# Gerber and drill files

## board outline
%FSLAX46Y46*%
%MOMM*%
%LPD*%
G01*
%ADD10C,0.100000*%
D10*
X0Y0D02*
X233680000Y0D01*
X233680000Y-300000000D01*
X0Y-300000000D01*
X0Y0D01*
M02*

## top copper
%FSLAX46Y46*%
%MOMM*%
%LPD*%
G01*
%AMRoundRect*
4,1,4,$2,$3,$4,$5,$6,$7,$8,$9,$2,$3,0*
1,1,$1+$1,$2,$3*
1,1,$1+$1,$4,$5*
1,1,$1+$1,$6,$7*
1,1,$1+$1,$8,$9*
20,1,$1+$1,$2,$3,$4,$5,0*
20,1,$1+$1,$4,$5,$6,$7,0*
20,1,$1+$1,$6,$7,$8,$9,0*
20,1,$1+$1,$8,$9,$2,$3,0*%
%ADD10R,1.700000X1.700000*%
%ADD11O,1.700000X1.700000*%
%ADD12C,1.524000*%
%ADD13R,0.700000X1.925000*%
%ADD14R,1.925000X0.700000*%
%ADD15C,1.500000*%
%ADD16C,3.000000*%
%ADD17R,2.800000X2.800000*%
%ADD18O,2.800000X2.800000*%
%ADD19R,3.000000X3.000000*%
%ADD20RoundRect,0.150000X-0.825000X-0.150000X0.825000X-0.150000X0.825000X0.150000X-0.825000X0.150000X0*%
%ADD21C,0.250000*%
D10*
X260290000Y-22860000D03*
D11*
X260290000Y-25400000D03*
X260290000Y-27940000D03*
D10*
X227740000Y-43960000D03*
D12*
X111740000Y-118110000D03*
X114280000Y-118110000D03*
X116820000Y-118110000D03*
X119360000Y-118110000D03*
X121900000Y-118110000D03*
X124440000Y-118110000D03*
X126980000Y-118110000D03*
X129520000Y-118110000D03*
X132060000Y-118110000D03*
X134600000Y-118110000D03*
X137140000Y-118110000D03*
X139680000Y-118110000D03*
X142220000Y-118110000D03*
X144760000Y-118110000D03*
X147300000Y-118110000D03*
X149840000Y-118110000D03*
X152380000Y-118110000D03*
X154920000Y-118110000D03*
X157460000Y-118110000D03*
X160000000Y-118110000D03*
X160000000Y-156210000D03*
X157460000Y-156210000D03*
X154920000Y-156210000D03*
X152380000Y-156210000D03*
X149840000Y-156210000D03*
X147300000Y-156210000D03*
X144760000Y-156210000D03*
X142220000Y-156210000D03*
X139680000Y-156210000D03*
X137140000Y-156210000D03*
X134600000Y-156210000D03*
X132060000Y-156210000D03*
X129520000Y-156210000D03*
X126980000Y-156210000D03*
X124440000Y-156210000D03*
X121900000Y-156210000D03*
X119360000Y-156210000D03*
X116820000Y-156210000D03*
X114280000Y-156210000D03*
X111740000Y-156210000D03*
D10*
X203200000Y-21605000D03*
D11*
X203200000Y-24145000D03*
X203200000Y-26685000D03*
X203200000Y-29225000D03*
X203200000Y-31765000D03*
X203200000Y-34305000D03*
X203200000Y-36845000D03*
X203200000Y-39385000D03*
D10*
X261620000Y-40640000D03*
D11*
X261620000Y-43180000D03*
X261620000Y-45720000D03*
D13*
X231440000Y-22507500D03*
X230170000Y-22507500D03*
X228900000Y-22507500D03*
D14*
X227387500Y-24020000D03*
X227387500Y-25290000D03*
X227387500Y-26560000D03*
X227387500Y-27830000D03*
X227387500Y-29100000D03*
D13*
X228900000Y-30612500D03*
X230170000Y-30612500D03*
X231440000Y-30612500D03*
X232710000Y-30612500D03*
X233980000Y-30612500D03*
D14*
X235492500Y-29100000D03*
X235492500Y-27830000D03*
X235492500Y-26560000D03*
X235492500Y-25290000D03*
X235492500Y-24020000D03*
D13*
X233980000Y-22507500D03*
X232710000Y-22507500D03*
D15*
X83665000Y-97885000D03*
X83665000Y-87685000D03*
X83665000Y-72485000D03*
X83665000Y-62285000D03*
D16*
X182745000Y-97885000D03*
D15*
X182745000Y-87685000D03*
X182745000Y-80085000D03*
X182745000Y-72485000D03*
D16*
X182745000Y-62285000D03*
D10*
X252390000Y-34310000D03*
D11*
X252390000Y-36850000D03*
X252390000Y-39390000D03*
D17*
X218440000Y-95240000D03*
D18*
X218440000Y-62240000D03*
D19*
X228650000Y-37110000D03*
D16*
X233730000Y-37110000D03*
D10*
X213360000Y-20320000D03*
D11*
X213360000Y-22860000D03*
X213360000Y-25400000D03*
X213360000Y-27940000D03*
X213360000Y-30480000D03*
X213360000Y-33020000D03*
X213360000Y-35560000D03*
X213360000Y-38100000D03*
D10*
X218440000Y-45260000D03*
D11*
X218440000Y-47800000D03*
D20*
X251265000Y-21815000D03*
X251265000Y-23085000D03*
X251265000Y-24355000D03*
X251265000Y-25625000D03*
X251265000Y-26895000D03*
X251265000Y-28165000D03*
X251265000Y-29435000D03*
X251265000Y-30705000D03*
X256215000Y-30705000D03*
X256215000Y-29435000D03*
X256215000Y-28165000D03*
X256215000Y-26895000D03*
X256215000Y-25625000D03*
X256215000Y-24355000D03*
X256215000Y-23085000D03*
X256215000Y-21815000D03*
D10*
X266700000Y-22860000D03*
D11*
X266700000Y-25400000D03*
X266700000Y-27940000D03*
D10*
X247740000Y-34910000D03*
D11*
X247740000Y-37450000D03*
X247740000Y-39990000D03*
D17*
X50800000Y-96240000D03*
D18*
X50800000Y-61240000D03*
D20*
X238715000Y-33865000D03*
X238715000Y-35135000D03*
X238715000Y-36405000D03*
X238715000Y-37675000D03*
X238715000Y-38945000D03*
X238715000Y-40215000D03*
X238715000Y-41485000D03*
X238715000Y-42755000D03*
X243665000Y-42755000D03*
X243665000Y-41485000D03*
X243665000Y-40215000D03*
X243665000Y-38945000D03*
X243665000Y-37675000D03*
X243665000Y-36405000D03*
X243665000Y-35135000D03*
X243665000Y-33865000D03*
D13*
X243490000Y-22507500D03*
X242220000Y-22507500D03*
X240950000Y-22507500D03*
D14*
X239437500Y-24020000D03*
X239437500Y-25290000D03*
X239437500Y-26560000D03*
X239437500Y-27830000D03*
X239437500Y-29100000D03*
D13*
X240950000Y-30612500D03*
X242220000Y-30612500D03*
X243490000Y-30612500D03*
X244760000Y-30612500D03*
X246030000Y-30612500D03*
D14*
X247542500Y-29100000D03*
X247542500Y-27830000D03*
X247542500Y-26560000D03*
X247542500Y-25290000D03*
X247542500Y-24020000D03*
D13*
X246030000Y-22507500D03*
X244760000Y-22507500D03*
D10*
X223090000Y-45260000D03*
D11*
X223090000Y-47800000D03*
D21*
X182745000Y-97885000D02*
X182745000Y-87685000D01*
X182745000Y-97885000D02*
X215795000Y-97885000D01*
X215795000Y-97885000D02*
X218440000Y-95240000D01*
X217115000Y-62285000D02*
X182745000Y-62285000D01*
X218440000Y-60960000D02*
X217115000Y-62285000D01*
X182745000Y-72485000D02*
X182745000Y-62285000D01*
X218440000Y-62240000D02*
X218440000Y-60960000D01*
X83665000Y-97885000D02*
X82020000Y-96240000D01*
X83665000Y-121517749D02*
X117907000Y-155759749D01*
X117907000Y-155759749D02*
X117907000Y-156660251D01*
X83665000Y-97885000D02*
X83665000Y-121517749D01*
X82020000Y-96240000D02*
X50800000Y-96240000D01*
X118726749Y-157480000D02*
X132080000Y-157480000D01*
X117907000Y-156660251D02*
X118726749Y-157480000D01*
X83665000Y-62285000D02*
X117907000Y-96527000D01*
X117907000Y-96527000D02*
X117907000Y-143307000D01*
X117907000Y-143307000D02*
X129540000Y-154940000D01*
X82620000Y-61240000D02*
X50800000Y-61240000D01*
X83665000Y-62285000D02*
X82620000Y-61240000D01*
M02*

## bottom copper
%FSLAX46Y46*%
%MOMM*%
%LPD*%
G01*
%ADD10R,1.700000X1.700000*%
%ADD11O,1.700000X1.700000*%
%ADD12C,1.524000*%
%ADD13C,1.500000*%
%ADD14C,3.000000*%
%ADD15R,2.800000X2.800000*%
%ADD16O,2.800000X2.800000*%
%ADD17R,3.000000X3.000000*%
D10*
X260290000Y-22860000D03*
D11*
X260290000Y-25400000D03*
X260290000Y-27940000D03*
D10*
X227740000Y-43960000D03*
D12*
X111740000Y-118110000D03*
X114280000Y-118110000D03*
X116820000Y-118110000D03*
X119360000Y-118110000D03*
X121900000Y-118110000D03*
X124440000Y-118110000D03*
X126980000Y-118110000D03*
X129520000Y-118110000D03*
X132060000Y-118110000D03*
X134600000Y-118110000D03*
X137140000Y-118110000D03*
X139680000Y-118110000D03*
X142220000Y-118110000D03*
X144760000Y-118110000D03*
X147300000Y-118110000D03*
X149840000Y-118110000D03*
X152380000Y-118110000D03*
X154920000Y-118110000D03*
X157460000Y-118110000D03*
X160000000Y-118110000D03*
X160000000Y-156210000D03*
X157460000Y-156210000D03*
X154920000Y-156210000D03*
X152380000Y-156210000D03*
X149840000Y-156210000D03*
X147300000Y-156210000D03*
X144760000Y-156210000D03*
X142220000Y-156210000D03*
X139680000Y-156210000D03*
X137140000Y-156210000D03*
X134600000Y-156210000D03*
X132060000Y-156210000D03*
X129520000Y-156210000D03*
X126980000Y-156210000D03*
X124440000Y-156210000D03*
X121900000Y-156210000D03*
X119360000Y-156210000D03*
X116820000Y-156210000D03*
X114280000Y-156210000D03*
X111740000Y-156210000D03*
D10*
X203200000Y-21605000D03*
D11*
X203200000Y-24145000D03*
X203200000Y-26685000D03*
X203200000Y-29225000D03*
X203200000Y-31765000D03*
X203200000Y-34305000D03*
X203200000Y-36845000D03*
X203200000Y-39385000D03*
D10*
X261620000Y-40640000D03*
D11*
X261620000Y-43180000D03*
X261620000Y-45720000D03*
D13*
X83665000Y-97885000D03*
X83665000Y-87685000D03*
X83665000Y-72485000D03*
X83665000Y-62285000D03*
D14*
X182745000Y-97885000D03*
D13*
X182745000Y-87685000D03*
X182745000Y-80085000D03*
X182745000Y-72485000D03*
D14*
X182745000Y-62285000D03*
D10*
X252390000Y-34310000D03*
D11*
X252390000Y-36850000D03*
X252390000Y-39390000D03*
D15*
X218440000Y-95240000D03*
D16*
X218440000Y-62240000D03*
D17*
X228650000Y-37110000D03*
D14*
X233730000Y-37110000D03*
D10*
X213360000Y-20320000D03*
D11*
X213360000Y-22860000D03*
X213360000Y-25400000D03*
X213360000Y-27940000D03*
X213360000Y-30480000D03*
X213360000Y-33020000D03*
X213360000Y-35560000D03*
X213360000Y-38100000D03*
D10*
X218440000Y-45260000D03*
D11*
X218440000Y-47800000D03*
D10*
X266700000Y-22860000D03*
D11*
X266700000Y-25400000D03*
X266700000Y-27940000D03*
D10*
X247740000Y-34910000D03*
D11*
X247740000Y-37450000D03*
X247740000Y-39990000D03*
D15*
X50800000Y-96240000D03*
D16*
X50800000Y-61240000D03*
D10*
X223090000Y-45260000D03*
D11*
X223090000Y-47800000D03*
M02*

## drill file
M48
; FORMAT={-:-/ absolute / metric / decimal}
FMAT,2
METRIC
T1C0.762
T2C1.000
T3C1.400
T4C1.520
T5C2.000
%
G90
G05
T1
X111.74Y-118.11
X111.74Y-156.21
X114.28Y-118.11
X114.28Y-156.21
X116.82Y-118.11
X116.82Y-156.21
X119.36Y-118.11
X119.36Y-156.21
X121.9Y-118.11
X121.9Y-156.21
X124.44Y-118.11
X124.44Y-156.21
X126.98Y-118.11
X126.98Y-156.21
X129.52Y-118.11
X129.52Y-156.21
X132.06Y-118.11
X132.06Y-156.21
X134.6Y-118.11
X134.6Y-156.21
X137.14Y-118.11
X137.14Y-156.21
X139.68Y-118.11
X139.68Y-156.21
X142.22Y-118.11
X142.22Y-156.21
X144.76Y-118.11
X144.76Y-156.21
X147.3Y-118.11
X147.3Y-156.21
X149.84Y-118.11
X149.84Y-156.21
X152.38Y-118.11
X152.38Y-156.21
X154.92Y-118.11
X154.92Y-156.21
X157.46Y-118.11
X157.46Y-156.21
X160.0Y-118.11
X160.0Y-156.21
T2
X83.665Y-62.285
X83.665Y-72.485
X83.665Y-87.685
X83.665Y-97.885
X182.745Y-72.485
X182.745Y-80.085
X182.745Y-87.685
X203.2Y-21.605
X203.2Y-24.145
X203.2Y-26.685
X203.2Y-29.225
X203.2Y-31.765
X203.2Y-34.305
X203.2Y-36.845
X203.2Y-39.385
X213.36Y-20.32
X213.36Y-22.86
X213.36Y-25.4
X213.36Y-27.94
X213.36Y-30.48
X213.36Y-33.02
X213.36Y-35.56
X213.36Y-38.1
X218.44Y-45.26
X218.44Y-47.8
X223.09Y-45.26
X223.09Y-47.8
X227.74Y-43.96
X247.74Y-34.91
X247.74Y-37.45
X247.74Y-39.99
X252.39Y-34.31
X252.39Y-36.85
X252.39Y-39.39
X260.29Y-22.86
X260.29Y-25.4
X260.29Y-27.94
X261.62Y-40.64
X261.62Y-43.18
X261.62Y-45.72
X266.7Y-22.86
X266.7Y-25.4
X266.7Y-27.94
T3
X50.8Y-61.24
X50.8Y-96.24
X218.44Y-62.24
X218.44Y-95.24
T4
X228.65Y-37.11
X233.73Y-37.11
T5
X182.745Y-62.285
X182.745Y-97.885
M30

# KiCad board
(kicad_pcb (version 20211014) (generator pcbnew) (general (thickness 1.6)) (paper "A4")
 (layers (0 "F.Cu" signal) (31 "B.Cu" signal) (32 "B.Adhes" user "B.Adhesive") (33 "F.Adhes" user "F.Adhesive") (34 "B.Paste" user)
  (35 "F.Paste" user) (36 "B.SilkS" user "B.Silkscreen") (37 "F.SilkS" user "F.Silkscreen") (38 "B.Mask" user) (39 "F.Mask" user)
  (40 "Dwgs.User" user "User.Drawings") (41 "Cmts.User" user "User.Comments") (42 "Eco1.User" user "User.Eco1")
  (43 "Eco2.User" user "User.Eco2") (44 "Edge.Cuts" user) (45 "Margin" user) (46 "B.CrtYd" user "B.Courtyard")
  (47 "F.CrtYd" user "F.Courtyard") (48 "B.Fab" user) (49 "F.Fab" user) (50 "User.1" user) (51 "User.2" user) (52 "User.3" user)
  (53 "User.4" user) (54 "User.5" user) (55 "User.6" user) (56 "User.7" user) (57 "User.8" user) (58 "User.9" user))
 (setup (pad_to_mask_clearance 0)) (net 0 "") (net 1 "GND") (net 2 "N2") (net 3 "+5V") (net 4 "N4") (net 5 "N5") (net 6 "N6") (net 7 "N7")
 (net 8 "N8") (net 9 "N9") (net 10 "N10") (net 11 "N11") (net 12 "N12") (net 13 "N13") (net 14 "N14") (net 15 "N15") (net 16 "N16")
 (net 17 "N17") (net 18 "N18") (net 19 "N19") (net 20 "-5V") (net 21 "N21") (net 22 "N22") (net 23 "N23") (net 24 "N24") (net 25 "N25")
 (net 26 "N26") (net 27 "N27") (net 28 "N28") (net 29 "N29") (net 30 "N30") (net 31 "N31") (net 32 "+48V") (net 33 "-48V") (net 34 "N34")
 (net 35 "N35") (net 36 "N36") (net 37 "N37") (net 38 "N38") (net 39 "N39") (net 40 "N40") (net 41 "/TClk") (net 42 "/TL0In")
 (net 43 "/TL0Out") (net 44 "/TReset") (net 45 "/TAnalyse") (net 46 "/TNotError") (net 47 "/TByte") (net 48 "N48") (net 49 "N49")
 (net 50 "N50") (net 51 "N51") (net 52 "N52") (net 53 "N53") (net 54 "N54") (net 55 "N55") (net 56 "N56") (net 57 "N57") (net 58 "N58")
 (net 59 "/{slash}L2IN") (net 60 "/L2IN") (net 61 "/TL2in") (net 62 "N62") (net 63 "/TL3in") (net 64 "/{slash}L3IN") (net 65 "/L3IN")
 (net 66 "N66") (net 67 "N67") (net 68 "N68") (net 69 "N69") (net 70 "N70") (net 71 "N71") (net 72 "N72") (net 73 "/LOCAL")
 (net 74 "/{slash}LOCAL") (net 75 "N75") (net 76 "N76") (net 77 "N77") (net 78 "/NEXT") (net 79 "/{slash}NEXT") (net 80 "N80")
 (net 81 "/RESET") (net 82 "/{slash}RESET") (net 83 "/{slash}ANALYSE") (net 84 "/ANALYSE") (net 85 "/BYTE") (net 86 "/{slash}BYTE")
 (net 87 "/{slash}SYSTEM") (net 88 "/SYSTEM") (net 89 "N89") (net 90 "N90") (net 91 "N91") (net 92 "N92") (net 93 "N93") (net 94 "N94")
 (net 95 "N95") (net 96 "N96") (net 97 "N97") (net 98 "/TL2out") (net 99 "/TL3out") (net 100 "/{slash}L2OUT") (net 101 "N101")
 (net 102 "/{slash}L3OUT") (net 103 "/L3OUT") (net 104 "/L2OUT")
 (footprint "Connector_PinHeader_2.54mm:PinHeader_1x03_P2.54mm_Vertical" (layer "F.Cu") (at 260.29 22.86)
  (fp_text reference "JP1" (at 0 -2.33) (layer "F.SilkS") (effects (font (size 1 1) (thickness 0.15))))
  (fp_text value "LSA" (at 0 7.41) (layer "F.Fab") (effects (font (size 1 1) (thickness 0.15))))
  (pad "1" thru_hole rect (at 0 0) (size 1.7 1.7) (drill 1) (layers *.Cu *.Mask) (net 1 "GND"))
  (pad "2" thru_hole oval (at 0 2.54) (size 1.7 1.7) (drill 1) (layers *.Cu *.Mask) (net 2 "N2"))
  (pad "3" thru_hole oval (at 0 5.08) (size 1.7 1.7) (drill 1) (layers *.Cu *.Mask) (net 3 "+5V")))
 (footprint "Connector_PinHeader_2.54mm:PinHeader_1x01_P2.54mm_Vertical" (layer "F.Cu") (at 227.74 43.96)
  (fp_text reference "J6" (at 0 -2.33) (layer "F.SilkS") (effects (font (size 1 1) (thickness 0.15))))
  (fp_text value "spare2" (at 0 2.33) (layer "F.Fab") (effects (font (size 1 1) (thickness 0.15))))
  (pad "1" thru_hole rect (at 0 0) (size 1.7 1.7) (drill 1) (layers *.Cu *.Mask) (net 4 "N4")))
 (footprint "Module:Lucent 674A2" (layer "F.Cu") (at 137.16 137.16)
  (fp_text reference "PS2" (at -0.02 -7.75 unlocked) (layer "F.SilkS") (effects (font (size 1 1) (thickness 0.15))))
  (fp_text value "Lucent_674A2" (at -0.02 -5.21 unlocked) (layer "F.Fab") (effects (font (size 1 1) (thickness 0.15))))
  (pad "1" thru_hole circle (at -25.42 -19.05) (size 1.524 1.524) (drill 0.762) (layers *.Cu *.Mask) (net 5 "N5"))
  (pad "2" thru_hole circle (at -22.88 -19.05) (size 1.524 1.524) (drill 0.762) (layers *.Cu *.Mask) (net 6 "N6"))
  (pad "3" thru_hole circle (at -20.34 -19.05) (size 1.524 1.524) (drill 0.762) (layers *.Cu *.Mask) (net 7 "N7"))
  (pad "4" thru_hole circle (at -17.8 -19.05) (size 1.524 1.524) (drill 0.762) (layers *.Cu *.Mask) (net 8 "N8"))
  (pad "5" thru_hole circle (at -15.26 -19.05) (size 1.524 1.524) (drill 0.762) (layers *.Cu *.Mask) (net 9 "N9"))
  (pad "6" thru_hole circle (at -12.72 -19.05) (size 1.524 1.524) (drill 0.762) (layers *.Cu *.Mask) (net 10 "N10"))
  (pad "7" thru_hole circle (at -10.18 -19.05) (size 1.524 1.524) (drill 0.762) (layers *.Cu *.Mask) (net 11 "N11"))
  (pad "8" thru_hole circle (at -7.64 -19.05) (size 1.524 1.524) (drill 0.762) (layers *.Cu *.Mask) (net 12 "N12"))
  (pad "9" thru_hole circle (at -5.1 -19.05) (size 1.524 1.524) (drill 0.762) (layers *.Cu *.Mask) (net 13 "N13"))
  (pad "10" thru_hole circle (at -2.56 -19.05) (size 1.524 1.524) (drill 0.762) (layers *.Cu *.Mask) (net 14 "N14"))
  (pad "11" thru_hole circle (at -0.02 -19.05) (size 1.524 1.524) (drill 0.762) (layers *.Cu *.Mask) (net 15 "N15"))
  (pad "12" thru_hole circle (at 2.52 -19.05) (size 1.524 1.524) (drill 0.762) (layers *.Cu *.Mask) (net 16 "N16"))
  (pad "13" thru_hole circle (at 5.06 -19.05) (size 1.524 1.524) (drill 0.762) (layers *.Cu *.Mask) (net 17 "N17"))
  (pad "14" thru_hole circle (at 7.6 -19.05) (size 1.524 1.524) (drill 0.762) (layers *.Cu *.Mask) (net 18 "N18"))
  (pad "15" thru_hole circle (at 10.14 -19.05) (size 1.524 1.524) (drill 0.762) (layers *.Cu *.Mask) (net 18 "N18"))
  (pad "16" thru_hole circle (at 12.68 -19.05) (size 1.524 1.524) (drill 0.762) (layers *.Cu *.Mask) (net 18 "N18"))
  (pad "17" thru_hole circle (at 15.22 -19.05) (size 1.524 1.524) (drill 0.762) (layers *.Cu *.Mask) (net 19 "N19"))
  (pad "18" thru_hole circle (at 17.76 -19.05) (size 1.524 1.524) (drill 0.762) (layers *.Cu *.Mask) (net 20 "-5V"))
  (pad "19" thru_hole circle (at 20.3 -19.05) (size 1.524 1.524) (drill 0.762) (layers *.Cu *.Mask) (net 20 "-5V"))
  (pad "20" thru_hole circle (at 22.84 -19.05) (size 1.524 1.524) (drill 0.762) (layers *.Cu *.Mask) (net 20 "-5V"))
  (pad "21" thru_hole circle (at 22.84 19.05) (size 1.524 1.524) (drill 0.762) (layers *.Cu *.Mask) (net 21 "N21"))
  (pad "22" thru_hole circle (at 20.3 19.05) (size 1.524 1.524) (drill 0.762) (layers *.Cu *.Mask) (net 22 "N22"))
  (pad "23" thru_hole circle (at 17.76 19.05) (size 1.524 1.524) (drill 0.762) (layers *.Cu *.Mask) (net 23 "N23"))
  (pad "24" thru_hole circle (at 15.22 19.05) (size 1.524 1.524) (drill 0.762) (layers *.Cu *.Mask) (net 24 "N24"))
  (pad "25" thru_hole circle (at 12.68 19.05) (size 1.524 1.524) (drill 0.762) (layers *.Cu *.Mask) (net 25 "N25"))
  (pad "26" thru_hole circle (at 10.14 19.05) (size 1.524 1.524) (drill 0.762) (layers *.Cu *.Mask) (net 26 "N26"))
  (pad "27" thru_hole circle (at 7.6 19.05) (size 1.524 1.524) (drill 0.762) (layers *.Cu *.Mask) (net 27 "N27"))
  (pad "28" thru_hole circle (at 5.06 19.05) (size 1.524 1.524) (drill 0.762) (layers *.Cu *.Mask) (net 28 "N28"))
  (pad "29" thru_hole circle (at 2.52 19.05) (size 1.524 1.524) (drill 0.762) (layers *.Cu *.Mask) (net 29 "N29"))
  (pad "30" thru_hole circle (at -0.02 19.05) (size 1.524 1.524) (drill 0.762) (layers *.Cu *.Mask) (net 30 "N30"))
  (pad "31" thru_hole circle (at -2.56 19.05) (size 1.524 1.524) (drill 0.762) (layers *.Cu *.Mask) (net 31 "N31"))
  (pad "32" thru_hole circle (at -5.1 19.05) (size 1.524 1.524) (drill 0.762) (layers *.Cu *.Mask) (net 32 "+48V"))
  (pad "33" thru_hole circle (at -7.64 19.05) (size 1.524 1.524) (drill 0.762) (layers *.Cu *.Mask) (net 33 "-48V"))
  (pad "34" thru_hole circle (at -10.18 19.05) (size 1.524 1.524) (drill 0.762) (layers *.Cu *.Mask) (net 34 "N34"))
  (pad "35" thru_hole circle (at -12.72 19.05) (size 1.524 1.524) (drill 0.762) (layers *.Cu *.Mask) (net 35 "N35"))
  (pad "36" thru_hole circle (at -15.26 19.05) (size 1.524 1.524) (drill 0.762) (layers *.Cu *.Mask) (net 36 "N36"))
  (pad "37" thru_hole circle (at -17.8 19.05) (size 1.524 1.524) (drill 0.762) (layers *.Cu *.Mask) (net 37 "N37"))
  (pad "38" thru_hole circle (at -20.34 19.05) (size 1.524 1.524) (drill 0.762) (layers *.Cu *.Mask) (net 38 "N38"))
  (pad "39" thru_hole circle (at -22.88 19.05) (size 1.524 1.524) (drill 0.762) (layers *.Cu *.Mask) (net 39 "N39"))
  (pad "40" thru_hole circle (at -25.42 19.05) (size 1.524 1.524) (drill 0.762) (layers *.Cu *.Mask) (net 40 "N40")))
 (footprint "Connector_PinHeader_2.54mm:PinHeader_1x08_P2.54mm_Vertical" (layer "F.Cu") (at 203.2 21.605)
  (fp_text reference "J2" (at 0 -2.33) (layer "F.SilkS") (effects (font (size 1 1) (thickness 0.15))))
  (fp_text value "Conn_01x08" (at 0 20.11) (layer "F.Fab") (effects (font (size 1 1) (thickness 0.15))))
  (pad "1" thru_hole rect (at 0 0) (size 1.7 1.7) (drill 1) (layers *.Cu *.Mask) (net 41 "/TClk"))
  (pad "2" thru_hole oval (at 0 2.54) (size 1.7 1.7) (drill 1) (layers *.Cu *.Mask) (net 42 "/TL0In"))
  (pad "3" thru_hole oval (at 0 5.08) (size 1.7 1.7) (drill 1) (layers *.Cu *.Mask) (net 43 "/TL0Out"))
  (pad "4" thru_hole oval (at 0 7.62) (size 1.7 1.7) (drill 1) (layers *.Cu *.Mask) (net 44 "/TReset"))
  (pad "5" thru_hole oval (at 0 10.16) (size 1.7 1.7) (drill 1) (layers *.Cu *.Mask) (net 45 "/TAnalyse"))
  (pad "6" thru_hole oval (at 0 12.7) (size 1.7 1.7) (drill 1) (layers *.Cu *.Mask) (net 1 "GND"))
  (pad "7" thru_hole oval (at 0 15.24) (size 1.7 1.7) (drill 1) (layers *.Cu *.Mask) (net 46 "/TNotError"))
  (pad "8" thru_hole oval (at 0 17.78) (size 1.7 1.7) (drill 1) (layers *.Cu *.Mask) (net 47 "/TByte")))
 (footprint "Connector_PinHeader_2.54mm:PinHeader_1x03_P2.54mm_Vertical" (layer "F.Cu") (at 261.62 40.64)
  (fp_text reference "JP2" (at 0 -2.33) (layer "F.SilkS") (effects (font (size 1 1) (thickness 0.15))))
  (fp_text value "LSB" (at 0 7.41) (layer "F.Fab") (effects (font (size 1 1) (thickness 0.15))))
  (pad "1" thru_hole rect (at 0 0) (size 1.7 1.7) (drill 1) (layers *.Cu *.Mask) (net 1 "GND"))
  (pad "2" thru_hole oval (at 0 2.54) (size 1.7 1.7) (drill 1) (layers *.Cu *.Mask) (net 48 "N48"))
  (pad "3" thru_hole oval (at 0 5.08) (size 1.7 1.7) (drill 1) (layers *.Cu *.Mask) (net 3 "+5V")))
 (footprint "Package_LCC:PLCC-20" (layer "F.Cu") (at 231.44 26.56)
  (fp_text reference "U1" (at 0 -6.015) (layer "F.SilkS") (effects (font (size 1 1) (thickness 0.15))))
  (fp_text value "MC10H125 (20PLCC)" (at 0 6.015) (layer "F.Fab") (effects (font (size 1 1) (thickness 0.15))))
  (pad "1" smd rect (at 0 -4.0525) (size 0.7 1.925) (layers "F.Cu" "F.Paste" "F.Mask") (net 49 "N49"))
  (pad "2" smd rect (at -1.27 -4.0525) (size 0.7 1.925) (layers "F.Cu" "F.Paste" "F.Mask") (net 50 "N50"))
  (pad "3" smd rect (at -2.54 -4.0525) (size 0.7 1.925) (layers "F.Cu" "F.Paste" "F.Mask") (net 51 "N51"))
  (pad "4" smd rect (at -4.0525 -2.54) (size 1.925 0.7) (layers "F.Cu" "F.Paste" "F.Mask") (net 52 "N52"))
  (pad "5" smd rect (at -4.0525 -1.27) (size 1.925 0.7) (layers "F.Cu" "F.Paste" "F.Mask") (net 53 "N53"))
  (pad "6" smd rect (at -4.0525 0) (size 1.925 0.7) (layers "F.Cu" "F.Paste" "F.Mask") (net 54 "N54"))
  (pad "7" smd rect (at -4.0525 1.27) (size 1.925 0.7) (layers "F.Cu" "F.Paste" "F.Mask") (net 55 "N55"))
  (pad "8" smd rect (at -4.0525 2.54) (size 1.925 0.7) (layers "F.Cu" "F.Paste" "F.Mask") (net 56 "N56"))
  (pad "9" smd rect (at -2.54 4.0525) (size 0.7 1.925) (layers "F.Cu" "F.Paste" "F.Mask") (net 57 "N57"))
  (pad "10" smd rect (at -1.27 4.0525) (size 0.7 1.925) (layers "F.Cu" "F.Paste" "F.Mask") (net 20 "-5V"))
  (pad "11" smd rect (at 0 4.0525) (size 0.7 1.925) (layers "F.Cu" "F.Paste" "F.Mask") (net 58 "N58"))
  (pad "12" smd rect (at 1.27 4.0525) (size 0.7 1.925) (layers "F.Cu" "F.Paste" "F.Mask") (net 3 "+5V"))
  (pad "13" smd rect (at 2.54 4.0525) (size 0.7 1.925) (layers "F.Cu" "F.Paste" "F.Mask") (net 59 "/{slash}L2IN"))
  (pad "14" smd rect (at 4.0525 2.54) (size 1.925 0.7) (layers "F.Cu" "F.Paste" "F.Mask") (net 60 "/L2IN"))
  (pad "15" smd rect (at 4.0525 1.27) (size 1.925 0.7) (layers "F.Cu" "F.Paste" "F.Mask") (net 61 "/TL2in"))
  (pad "16" smd rect (at 4.0525 0) (size 1.925 0.7) (layers "F.Cu" "F.Paste" "F.Mask") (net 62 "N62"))
  (pad "17" smd rect (at 4.0525 -1.27) (size 1.925 0.7) (layers "F.Cu" "F.Paste" "F.Mask") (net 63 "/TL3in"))
  (pad "18" smd rect (at 4.0525 -2.54) (size 1.925 0.7) (layers "F.Cu" "F.Paste" "F.Mask") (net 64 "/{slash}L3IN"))
  (pad "19" smd rect (at 2.54 -4.0525) (size 0.7 1.925) (layers "F.Cu" "F.Paste" "F.Mask") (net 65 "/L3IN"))
  (pad "20" smd rect (at 1.27 -4.0525) (size 0.7 1.925) (layers "F.Cu" "F.Paste" "F.Mask") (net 1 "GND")))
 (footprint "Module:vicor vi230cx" (layer "F.Cu") (at 76.065 49.585)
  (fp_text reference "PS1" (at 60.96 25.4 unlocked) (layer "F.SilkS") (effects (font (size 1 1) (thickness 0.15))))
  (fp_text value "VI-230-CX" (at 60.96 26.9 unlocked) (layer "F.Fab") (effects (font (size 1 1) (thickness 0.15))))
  (pad "1" thru_hole circle (at 7.6 48.3) (size 1.5 1.5) (drill 1) (layers *.Cu *.Mask) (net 32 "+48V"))
  (pad "2" thru_hole circle (at 7.6 38.1) (size 1.5 1.5) (drill 1) (layers *.Cu *.Mask) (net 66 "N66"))
  (pad "3" thru_hole circle (at 7.6 22.9) (size 1.5 1.5) (drill 1) (layers *.Cu *.Mask) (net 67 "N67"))
  (pad "4" thru_hole circle (at 7.6 12.7) (size 1.5 1.5) (drill 1) (layers *.Cu *.Mask) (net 33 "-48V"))
  (pad "5" thru_hole circle (at 106.68 48.3) (size 3 3) (drill 2) (layers *.Cu *.Mask) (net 3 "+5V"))
  (pad "6" thru_hole circle (at 106.68 38.1) (size 1.5 1.5) (drill 1) (layers *.Cu *.Mask) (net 3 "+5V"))
  (pad "7" thru_hole circle (at 106.68 30.5) (size 1.5 1.5) (drill 1) (layers *.Cu *.Mask) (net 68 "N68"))
  (pad "8" thru_hole circle (at 106.68 22.9) (size 1.5 1.5) (drill 1) (layers *.Cu *.Mask) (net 1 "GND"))
  (pad "9" thru_hole circle (at 106.68 12.7) (size 3 3) (drill 2) (layers *.Cu *.Mask) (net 1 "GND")))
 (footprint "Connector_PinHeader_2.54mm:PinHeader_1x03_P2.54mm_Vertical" (layer "F.Cu") (at 252.39 34.31)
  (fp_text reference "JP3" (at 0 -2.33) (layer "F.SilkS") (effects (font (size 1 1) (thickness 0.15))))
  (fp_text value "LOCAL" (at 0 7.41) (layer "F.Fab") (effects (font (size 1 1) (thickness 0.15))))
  (pad "1" thru_hole rect (at 0 0) (size 1.7 1.7) (drill 1) (layers *.Cu *.Mask) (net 1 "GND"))
  (pad "2" thru_hole oval (at 0 2.54) (size 1.7 1.7) (drill 1) (layers *.Cu *.Mask) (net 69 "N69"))
  (pad "3" thru_hole oval (at 0 5.08) (size 1.7 1.7) (drill 1) (layers *.Cu *.Mask) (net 3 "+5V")))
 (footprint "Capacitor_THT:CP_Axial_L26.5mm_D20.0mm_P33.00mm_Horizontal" (layer "F.Cu") (at 218.44 95.24 90)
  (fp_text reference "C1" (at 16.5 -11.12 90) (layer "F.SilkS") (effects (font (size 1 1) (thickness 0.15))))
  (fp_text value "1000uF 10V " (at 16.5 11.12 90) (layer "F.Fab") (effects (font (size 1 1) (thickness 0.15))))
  (pad "1" thru_hole rect (at 0 0 90) (size 2.8 2.8) (drill 1.4) (layers *.Cu *.Mask) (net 3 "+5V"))
  (pad "2" thru_hole oval (at 33 0 90) (size 2.8 2.8) (drill 1.4) (layers *.Cu *.Mask) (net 1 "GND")))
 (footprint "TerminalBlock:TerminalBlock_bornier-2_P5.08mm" (layer "F.Cu") (at 228.65 37.11)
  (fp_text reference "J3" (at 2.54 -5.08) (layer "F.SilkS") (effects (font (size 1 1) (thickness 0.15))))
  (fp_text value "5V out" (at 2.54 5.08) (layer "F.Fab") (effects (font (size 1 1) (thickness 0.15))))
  (pad "1" thru_hole rect (at 0 0) (size 3 3) (drill 1.52) (layers *.Cu *.Mask) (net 1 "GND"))
  (pad "2" thru_hole circle (at 5.08 0) (size 3 3) (drill 1.52) (layers *.Cu *.Mask) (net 3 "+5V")))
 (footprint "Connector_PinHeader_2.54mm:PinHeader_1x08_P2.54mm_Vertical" (layer "F.Cu") (at 213.36 20.32)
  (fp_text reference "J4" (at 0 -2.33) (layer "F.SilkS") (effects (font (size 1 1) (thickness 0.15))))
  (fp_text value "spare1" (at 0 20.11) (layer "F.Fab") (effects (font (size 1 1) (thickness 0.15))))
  (pad "1" thru_hole rect (at 0 0) (size 1.7 1.7) (drill 1) (layers *.Cu *.Mask) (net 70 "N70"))
  (pad "2" thru_hole oval (at 0 2.54) (size 1.7 1.7) (drill 1) (layers *.Cu *.Mask))
  (pad "3" thru_hole oval (at 0 5.08) (size 1.7 1.7) (drill 1) (layers *.Cu *.Mask))
  (pad "4" thru_hole oval (at 0 7.62) (size 1.7 1.7) (drill 1) (layers *.Cu *.Mask))
  (pad "5" thru_hole oval (at 0 10.16) (size 1.7 1.7) (drill 1) (layers *.Cu *.Mask))
  (pad "6" thru_hole oval (at 0 12.7) (size 1.7 1.7) (drill 1) (layers *.Cu *.Mask))
  (pad "7" thru_hole oval (at 0 15.24) (size 1.7 1.7) (drill 1) (layers *.Cu *.Mask))
  (pad "8" thru_hole oval (at 0 17.78) (size 1.7 1.7) (drill 1) (layers *.Cu *.Mask)))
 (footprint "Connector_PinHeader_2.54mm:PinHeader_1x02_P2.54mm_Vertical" (layer "F.Cu") (at 218.44 45.26)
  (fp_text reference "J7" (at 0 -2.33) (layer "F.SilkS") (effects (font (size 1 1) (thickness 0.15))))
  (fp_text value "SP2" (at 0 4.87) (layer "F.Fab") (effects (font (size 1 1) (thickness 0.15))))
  (pad "1" thru_hole rect (at 0 0) (size 1.7 1.7) (drill 1) (layers *.Cu *.Mask) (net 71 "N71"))
  (pad "2" thru_hole oval (at 0 2.54) (size 1.7 1.7) (drill 1) (layers *.Cu *.Mask) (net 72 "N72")))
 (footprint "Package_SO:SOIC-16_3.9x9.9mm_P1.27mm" (layer "F.Cu") (at 253.74 26.26)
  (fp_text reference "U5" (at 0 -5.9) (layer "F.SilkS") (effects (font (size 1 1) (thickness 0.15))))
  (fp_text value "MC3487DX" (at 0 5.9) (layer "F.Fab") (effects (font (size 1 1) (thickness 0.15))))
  (pad "1" smd roundrect (at -2.475 -4.445) (size 1.95 0.6) (layers "F.Cu" "F.Paste" "F.Mask") (roundrect_rratio 0.25) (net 69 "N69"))
  (pad "2" smd roundrect (at -2.475 -3.175) (size 1.95 0.6) (layers "F.Cu" "F.Paste" "F.Mask") (roundrect_rratio 0.25) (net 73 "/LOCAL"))
  (pad "3" smd roundrect (at -2.475 -1.905) (size 1.95 0.6) (layers "F.Cu" "F.Paste" "F.Mask") (roundrect_rratio 0.25)
   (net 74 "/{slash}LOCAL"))
  (pad "4" smd roundrect (at -2.475 -0.635) (size 1.95 0.6) (layers "F.Cu" "F.Paste" "F.Mask") (roundrect_rratio 0.25) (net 3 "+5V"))
  (pad "5" smd roundrect (at -2.475 0.635) (size 1.95 0.6) (layers "F.Cu" "F.Paste" "F.Mask") (roundrect_rratio 0.25) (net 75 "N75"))
  (pad "6" smd roundrect (at -2.475 1.905) (size 1.95 0.6) (layers "F.Cu" "F.Paste" "F.Mask") (roundrect_rratio 0.25) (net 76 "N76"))
  (pad "7" smd roundrect (at -2.475 3.175) (size 1.95 0.6) (layers "F.Cu" "F.Paste" "F.Mask") (roundrect_rratio 0.25) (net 70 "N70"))
  (pad "8" smd roundrect (at -2.475 4.445) (size 1.95 0.6) (layers "F.Cu" "F.Paste" "F.Mask") (roundrect_rratio 0.25) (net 1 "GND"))
  (pad "9" smd roundrect (at 2.475 4.445) (size 1.95 0.6) (layers "F.Cu" "F.Paste" "F.Mask") (roundrect_rratio 0.25) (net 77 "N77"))
  (pad "10" smd roundrect (at 2.475 3.175) (size 1.95 0.6) (layers "F.Cu" "F.Paste" "F.Mask") (roundrect_rratio 0.25) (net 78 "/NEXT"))
  (pad "11" smd roundrect (at 2.475 1.905) (size 1.95 0.6) (layers "F.Cu" "F.Paste" "F.Mask") (roundrect_rratio 0.25)
   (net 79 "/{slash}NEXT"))
  (pad "12" smd roundrect (at 2.475 0.635) (size 1.95 0.6) (layers "F.Cu" "F.Paste" "F.Mask") (roundrect_rratio 0.25) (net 3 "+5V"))
  (pad "13" smd roundrect (at 2.475 -0.635) (size 1.95 0.6) (layers "F.Cu" "F.Paste" "F.Mask") (roundrect_rratio 0.25) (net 71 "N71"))
  (pad "14" smd roundrect (at 2.475 -1.905) (size 1.95 0.6) (layers "F.Cu" "F.Paste" "F.Mask") (roundrect_rratio 0.25) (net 72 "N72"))
  (pad "15" smd roundrect (at 2.475 -3.175) (size 1.95 0.6) (layers "F.Cu" "F.Paste" "F.Mask") (roundrect_rratio 0.25) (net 4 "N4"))
  (pad "16" smd roundrect (at 2.475 -4.445) (size 1.95 0.6) (layers "F.Cu" "F.Paste" "F.Mask") (roundrect_rratio 0.25) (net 3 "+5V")))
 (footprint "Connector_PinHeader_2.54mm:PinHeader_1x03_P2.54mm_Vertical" (layer "F.Cu") (at 266.7 22.86)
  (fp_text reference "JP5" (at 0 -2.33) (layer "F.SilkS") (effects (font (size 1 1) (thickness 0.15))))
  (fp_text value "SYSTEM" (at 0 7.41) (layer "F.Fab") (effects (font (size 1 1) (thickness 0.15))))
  (pad "1" thru_hole rect (at 0 0) (size 1.7 1.7) (drill 1) (layers *.Cu *.Mask) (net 1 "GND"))
  (pad "2" thru_hole oval (at 0 2.54) (size 1.7 1.7) (drill 1) (layers *.Cu *.Mask) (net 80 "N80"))
  (pad "3" thru_hole oval (at 0 5.08) (size 1.7 1.7) (drill 1) (layers *.Cu *.Mask) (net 3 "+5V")))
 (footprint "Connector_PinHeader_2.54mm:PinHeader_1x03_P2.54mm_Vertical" (layer "F.Cu") (at 247.74 34.91)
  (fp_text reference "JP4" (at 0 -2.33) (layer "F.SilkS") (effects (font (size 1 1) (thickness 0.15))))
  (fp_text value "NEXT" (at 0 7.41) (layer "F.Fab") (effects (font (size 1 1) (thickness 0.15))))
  (pad "1" thru_hole rect (at 0 0) (size 1.7 1.7) (drill 1) (layers *.Cu *.Mask) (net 1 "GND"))
  (pad "2" thru_hole oval (at 0 2.54) (size 1.7 1.7) (drill 1) (layers *.Cu *.Mask) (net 77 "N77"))
  (pad "3" thru_hole oval (at 0 5.08) (size 1.7 1.7) (drill 1) (layers *.Cu *.Mask) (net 3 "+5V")))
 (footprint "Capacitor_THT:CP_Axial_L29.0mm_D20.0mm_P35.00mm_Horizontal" (layer "F.Cu") (at 50.8 96.24 90)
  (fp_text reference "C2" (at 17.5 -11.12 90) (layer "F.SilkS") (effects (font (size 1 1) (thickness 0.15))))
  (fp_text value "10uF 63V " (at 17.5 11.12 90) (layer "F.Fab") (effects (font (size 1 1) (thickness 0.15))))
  (pad "1" thru_hole rect (at 0 0 90) (size 2.8 2.8) (drill 1.4) (layers *.Cu *.Mask) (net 32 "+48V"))
  (pad "2" thru_hole oval (at 35 0 90) (size 2.8 2.8) (drill 1.4) (layers *.Cu *.Mask) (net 33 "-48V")))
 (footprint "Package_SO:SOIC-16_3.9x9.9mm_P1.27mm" (layer "F.Cu") (at 241.19 38.31)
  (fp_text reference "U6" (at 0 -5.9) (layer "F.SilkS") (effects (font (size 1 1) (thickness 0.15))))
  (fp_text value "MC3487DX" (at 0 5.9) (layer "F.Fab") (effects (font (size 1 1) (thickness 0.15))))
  (pad "1" smd roundrect (at -2.475 -4.445) (size 1.95 0.6) (layers "F.Cu" "F.Paste" "F.Mask") (roundrect_rratio 0.25) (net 44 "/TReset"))
  (pad "2" smd roundrect (at -2.475 -3.175) (size 1.95 0.6) (layers "F.Cu" "F.Paste" "F.Mask") (roundrect_rratio 0.25) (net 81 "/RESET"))
  (pad "3" smd roundrect (at -2.475 -1.905) (size 1.95 0.6) (layers "F.Cu" "F.Paste" "F.Mask") (roundrect_rratio 0.25)
   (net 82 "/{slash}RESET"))
  (pad "4" smd roundrect (at -2.475 -0.635) (size 1.95 0.6) (layers "F.Cu" "F.Paste" "F.Mask") (roundrect_rratio 0.25) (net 3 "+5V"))
  (pad "5" smd roundrect (at -2.475 0.635) (size 1.95 0.6) (layers "F.Cu" "F.Paste" "F.Mask") (roundrect_rratio 0.25)
   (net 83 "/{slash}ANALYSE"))
  (pad "6" smd roundrect (at -2.475 1.905) (size 1.95 0.6) (layers "F.Cu" "F.Paste" "F.Mask") (roundrect_rratio 0.25) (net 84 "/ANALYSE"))
  (pad "7" smd roundrect (at -2.475 3.175) (size 1.95 0.6) (layers "F.Cu" "F.Paste" "F.Mask") (roundrect_rratio 0.25) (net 45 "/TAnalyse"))
  (pad "8" smd roundrect (at -2.475 4.445) (size 1.95 0.6) (layers "F.Cu" "F.Paste" "F.Mask") (roundrect_rratio 0.25) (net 1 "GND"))
  (pad "9" smd roundrect (at 2.475 4.445) (size 1.95 0.6) (layers "F.Cu" "F.Paste" "F.Mask") (roundrect_rratio 0.25) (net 47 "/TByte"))
  (pad "10" smd roundrect (at 2.475 3.175) (size 1.95 0.6) (layers "F.Cu" "F.Paste" "F.Mask") (roundrect_rratio 0.25) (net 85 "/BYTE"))
  (pad "11" smd roundrect (at 2.475 1.905) (size 1.95 0.6) (layers "F.Cu" "F.Paste" "F.Mask") (roundrect_rratio 0.25)
   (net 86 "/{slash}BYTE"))
  (pad "12" smd roundrect (at 2.475 0.635) (size 1.95 0.6) (layers "F.Cu" "F.Paste" "F.Mask") (roundrect_rratio 0.25) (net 3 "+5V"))
  (pad "13" smd roundrect (at 2.475 -0.635) (size 1.95 0.6) (layers "F.Cu" "F.Paste" "F.Mask") (roundrect_rratio 0.25)
   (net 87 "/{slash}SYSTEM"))
  (pad "14" smd roundrect (at 2.475 -1.905) (size 1.95 0.6) (layers "F.Cu" "F.Paste" "F.Mask") (roundrect_rratio 0.25) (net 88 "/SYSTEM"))
  (pad "15" smd roundrect (at 2.475 -3.175) (size 1.95 0.6) (layers "F.Cu" "F.Paste" "F.Mask") (roundrect_rratio 0.25) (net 80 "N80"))
  (pad "16" smd roundrect (at 2.475 -4.445) (size 1.95 0.6) (layers "F.Cu" "F.Paste" "F.Mask") (roundrect_rratio 0.25) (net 3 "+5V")))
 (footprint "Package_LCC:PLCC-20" (layer "F.Cu") (at 243.49 26.56)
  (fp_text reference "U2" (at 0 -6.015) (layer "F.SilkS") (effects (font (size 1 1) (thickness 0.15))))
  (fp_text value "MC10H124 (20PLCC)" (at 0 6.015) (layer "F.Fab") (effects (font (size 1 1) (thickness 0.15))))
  (pad "1" smd rect (at 0 -4.0525) (size 0.7 1.925) (layers "F.Cu" "F.Paste" "F.Mask") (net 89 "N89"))
  (pad "2" smd rect (at -1.27 -4.0525) (size 0.7 1.925) (layers "F.Cu" "F.Paste" "F.Mask") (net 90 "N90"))
  (pad "3" smd rect (at -2.54 -4.0525) (size 0.7 1.925) (layers "F.Cu" "F.Paste" "F.Mask") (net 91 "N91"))
  (pad "4" smd rect (at -4.0525 -2.54) (size 1.925 0.7) (layers "F.Cu" "F.Paste" "F.Mask") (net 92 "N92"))
  (pad "5" smd rect (at -4.0525 -1.27) (size 1.925 0.7) (layers "F.Cu" "F.Paste" "F.Mask") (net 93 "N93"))
  (pad "6" smd rect (at -4.0525 0) (size 1.925 0.7) (layers "F.Cu" "F.Paste" "F.Mask") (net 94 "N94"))
  (pad "7" smd rect (at -4.0525 1.27) (size 1.925 0.7) (layers "F.Cu" "F.Paste" "F.Mask") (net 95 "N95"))
  (pad "8" smd rect (at -4.0525 2.54) (size 1.925 0.7) (layers "F.Cu" "F.Paste" "F.Mask") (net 3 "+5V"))
  (pad "9" smd rect (at -2.54 4.0525) (size 0.7 1.925) (layers "F.Cu" "F.Paste" "F.Mask") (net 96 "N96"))
  (pad "10" smd rect (at -1.27 4.0525) (size 0.7 1.925) (layers "F.Cu" "F.Paste" "F.Mask") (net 20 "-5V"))
  (pad "11" smd rect (at 0 4.0525) (size 0.7 1.925) (layers "F.Cu" "F.Paste" "F.Mask") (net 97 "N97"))
  (pad "12" smd rect (at 1.27 4.0525) (size 0.7 1.925) (layers "F.Cu" "F.Paste" "F.Mask") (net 3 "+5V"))
  (pad "13" smd rect (at 2.54 4.0525) (size 0.7 1.925) (layers "F.Cu" "F.Paste" "F.Mask") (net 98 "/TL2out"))
  (pad "14" smd rect (at 4.0525 2.54) (size 1.925 0.7) (layers "F.Cu" "F.Paste" "F.Mask") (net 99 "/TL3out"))
  (pad "15" smd rect (at 4.0525 1.27) (size 1.925 0.7) (layers "F.Cu" "F.Paste" "F.Mask") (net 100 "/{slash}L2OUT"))
  (pad "16" smd rect (at 4.0525 0) (size 1.925 0.7) (layers "F.Cu" "F.Paste" "F.Mask") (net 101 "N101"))
  (pad "17" smd rect (at 4.0525 -1.27) (size 1.925 0.7) (layers "F.Cu" "F.Paste" "F.Mask") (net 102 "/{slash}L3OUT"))
  (pad "18" smd rect (at 4.0525 -2.54) (size 1.925 0.7) (layers "F.Cu" "F.Paste" "F.Mask") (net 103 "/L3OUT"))
  (pad "19" smd rect (at 2.54 -4.0525) (size 0.7 1.925) (layers "F.Cu" "F.Paste" "F.Mask") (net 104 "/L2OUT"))
  (pad "20" smd rect (at 1.27 -4.0525) (size 0.7 1.925) (layers "F.Cu" "F.Paste" "F.Mask") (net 1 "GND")))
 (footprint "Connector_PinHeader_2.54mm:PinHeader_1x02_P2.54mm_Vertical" (layer "F.Cu") (at 223.09 45.26)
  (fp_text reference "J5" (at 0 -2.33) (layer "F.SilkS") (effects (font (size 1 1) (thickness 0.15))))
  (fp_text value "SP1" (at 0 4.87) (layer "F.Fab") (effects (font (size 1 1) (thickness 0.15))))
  (pad "1" thru_hole rect (at 0 0) (size 1.7 1.7) (drill 1) (layers *.Cu *.Mask) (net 75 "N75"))
  (pad "2" thru_hole oval (at 0 2.54) (size 1.7 1.7) (drill 1) (layers *.Cu *.Mask) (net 76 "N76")))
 (gr_rect (start 0 0) (end 233.68 300) (layer "Edge.Cuts") (width 0.1) (fill none))
 (segment (start 182.745 97.885) (end 182.745 87.685) (width 0.25) (layer "F.Cu") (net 3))
 (segment (start 182.745 97.885) (end 215.795 97.885) (width 0.25) (layer "F.Cu") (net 3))
 (segment (start 215.795 97.885) (end 218.44 95.24) (width 0.25) (layer "F.Cu") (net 3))
 (segment (start 217.115 62.285) (end 182.745 62.285) (width 0.25) (layer "F.Cu") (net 1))
 (segment (start 218.44 60.96) (end 217.115 62.285) (width 0.25) (layer "F.Cu") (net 1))
 (segment (start 182.745 72.485) (end 182.745 62.285) (width 0.25) (layer "F.Cu") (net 1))
 (segment (start 218.44 62.24) (end 218.44 60.96) (width 0.25) (layer "F.Cu") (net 1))
 (segment (start 83.665 97.885) (end 82.02 96.24) (width 0.25) (layer "F.Cu") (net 32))
 (segment (start 83.665 121.517749) (end 117.907 155.759749) (width 0.25) (layer "F.Cu") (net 32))
 (segment (start 117.907 155.759749) (end 117.907 156.660251) (width 0.25) (layer "F.Cu") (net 32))
 (segment (start 83.665 97.885) (end 83.665 121.517749) (width 0.25) (layer "F.Cu") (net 32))
 (segment (start 82.02 96.24) (end 50.8 96.24) (width 0.25) (layer "F.Cu") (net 32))
 (segment (start 118.726749 157.48) (end 132.08 157.48) (width 0.25) (layer "F.Cu") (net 32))
 (segment (start 117.907 156.660251) (end 118.726749 157.48) (width 0.25) (layer "F.Cu") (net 32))
 (segment (start 83.665 62.285) (end 117.907 96.527) (width 0.25) (layer "F.Cu") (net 33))
 (segment (start 117.907 96.527) (end 117.907 143.307) (width 0.25) (layer "F.Cu") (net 33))
 (segment (start 117.907 143.307) (end 129.54 154.94) (width 0.25) (layer "F.Cu") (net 33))
 (segment (start 82.62 61.24) (end 50.8 61.24) (width 0.25) (layer "F.Cu") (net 33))
 (segment (start 83.665 62.285) (end 82.62 61.24) (width 0.25) (layer "F.Cu") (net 33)))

